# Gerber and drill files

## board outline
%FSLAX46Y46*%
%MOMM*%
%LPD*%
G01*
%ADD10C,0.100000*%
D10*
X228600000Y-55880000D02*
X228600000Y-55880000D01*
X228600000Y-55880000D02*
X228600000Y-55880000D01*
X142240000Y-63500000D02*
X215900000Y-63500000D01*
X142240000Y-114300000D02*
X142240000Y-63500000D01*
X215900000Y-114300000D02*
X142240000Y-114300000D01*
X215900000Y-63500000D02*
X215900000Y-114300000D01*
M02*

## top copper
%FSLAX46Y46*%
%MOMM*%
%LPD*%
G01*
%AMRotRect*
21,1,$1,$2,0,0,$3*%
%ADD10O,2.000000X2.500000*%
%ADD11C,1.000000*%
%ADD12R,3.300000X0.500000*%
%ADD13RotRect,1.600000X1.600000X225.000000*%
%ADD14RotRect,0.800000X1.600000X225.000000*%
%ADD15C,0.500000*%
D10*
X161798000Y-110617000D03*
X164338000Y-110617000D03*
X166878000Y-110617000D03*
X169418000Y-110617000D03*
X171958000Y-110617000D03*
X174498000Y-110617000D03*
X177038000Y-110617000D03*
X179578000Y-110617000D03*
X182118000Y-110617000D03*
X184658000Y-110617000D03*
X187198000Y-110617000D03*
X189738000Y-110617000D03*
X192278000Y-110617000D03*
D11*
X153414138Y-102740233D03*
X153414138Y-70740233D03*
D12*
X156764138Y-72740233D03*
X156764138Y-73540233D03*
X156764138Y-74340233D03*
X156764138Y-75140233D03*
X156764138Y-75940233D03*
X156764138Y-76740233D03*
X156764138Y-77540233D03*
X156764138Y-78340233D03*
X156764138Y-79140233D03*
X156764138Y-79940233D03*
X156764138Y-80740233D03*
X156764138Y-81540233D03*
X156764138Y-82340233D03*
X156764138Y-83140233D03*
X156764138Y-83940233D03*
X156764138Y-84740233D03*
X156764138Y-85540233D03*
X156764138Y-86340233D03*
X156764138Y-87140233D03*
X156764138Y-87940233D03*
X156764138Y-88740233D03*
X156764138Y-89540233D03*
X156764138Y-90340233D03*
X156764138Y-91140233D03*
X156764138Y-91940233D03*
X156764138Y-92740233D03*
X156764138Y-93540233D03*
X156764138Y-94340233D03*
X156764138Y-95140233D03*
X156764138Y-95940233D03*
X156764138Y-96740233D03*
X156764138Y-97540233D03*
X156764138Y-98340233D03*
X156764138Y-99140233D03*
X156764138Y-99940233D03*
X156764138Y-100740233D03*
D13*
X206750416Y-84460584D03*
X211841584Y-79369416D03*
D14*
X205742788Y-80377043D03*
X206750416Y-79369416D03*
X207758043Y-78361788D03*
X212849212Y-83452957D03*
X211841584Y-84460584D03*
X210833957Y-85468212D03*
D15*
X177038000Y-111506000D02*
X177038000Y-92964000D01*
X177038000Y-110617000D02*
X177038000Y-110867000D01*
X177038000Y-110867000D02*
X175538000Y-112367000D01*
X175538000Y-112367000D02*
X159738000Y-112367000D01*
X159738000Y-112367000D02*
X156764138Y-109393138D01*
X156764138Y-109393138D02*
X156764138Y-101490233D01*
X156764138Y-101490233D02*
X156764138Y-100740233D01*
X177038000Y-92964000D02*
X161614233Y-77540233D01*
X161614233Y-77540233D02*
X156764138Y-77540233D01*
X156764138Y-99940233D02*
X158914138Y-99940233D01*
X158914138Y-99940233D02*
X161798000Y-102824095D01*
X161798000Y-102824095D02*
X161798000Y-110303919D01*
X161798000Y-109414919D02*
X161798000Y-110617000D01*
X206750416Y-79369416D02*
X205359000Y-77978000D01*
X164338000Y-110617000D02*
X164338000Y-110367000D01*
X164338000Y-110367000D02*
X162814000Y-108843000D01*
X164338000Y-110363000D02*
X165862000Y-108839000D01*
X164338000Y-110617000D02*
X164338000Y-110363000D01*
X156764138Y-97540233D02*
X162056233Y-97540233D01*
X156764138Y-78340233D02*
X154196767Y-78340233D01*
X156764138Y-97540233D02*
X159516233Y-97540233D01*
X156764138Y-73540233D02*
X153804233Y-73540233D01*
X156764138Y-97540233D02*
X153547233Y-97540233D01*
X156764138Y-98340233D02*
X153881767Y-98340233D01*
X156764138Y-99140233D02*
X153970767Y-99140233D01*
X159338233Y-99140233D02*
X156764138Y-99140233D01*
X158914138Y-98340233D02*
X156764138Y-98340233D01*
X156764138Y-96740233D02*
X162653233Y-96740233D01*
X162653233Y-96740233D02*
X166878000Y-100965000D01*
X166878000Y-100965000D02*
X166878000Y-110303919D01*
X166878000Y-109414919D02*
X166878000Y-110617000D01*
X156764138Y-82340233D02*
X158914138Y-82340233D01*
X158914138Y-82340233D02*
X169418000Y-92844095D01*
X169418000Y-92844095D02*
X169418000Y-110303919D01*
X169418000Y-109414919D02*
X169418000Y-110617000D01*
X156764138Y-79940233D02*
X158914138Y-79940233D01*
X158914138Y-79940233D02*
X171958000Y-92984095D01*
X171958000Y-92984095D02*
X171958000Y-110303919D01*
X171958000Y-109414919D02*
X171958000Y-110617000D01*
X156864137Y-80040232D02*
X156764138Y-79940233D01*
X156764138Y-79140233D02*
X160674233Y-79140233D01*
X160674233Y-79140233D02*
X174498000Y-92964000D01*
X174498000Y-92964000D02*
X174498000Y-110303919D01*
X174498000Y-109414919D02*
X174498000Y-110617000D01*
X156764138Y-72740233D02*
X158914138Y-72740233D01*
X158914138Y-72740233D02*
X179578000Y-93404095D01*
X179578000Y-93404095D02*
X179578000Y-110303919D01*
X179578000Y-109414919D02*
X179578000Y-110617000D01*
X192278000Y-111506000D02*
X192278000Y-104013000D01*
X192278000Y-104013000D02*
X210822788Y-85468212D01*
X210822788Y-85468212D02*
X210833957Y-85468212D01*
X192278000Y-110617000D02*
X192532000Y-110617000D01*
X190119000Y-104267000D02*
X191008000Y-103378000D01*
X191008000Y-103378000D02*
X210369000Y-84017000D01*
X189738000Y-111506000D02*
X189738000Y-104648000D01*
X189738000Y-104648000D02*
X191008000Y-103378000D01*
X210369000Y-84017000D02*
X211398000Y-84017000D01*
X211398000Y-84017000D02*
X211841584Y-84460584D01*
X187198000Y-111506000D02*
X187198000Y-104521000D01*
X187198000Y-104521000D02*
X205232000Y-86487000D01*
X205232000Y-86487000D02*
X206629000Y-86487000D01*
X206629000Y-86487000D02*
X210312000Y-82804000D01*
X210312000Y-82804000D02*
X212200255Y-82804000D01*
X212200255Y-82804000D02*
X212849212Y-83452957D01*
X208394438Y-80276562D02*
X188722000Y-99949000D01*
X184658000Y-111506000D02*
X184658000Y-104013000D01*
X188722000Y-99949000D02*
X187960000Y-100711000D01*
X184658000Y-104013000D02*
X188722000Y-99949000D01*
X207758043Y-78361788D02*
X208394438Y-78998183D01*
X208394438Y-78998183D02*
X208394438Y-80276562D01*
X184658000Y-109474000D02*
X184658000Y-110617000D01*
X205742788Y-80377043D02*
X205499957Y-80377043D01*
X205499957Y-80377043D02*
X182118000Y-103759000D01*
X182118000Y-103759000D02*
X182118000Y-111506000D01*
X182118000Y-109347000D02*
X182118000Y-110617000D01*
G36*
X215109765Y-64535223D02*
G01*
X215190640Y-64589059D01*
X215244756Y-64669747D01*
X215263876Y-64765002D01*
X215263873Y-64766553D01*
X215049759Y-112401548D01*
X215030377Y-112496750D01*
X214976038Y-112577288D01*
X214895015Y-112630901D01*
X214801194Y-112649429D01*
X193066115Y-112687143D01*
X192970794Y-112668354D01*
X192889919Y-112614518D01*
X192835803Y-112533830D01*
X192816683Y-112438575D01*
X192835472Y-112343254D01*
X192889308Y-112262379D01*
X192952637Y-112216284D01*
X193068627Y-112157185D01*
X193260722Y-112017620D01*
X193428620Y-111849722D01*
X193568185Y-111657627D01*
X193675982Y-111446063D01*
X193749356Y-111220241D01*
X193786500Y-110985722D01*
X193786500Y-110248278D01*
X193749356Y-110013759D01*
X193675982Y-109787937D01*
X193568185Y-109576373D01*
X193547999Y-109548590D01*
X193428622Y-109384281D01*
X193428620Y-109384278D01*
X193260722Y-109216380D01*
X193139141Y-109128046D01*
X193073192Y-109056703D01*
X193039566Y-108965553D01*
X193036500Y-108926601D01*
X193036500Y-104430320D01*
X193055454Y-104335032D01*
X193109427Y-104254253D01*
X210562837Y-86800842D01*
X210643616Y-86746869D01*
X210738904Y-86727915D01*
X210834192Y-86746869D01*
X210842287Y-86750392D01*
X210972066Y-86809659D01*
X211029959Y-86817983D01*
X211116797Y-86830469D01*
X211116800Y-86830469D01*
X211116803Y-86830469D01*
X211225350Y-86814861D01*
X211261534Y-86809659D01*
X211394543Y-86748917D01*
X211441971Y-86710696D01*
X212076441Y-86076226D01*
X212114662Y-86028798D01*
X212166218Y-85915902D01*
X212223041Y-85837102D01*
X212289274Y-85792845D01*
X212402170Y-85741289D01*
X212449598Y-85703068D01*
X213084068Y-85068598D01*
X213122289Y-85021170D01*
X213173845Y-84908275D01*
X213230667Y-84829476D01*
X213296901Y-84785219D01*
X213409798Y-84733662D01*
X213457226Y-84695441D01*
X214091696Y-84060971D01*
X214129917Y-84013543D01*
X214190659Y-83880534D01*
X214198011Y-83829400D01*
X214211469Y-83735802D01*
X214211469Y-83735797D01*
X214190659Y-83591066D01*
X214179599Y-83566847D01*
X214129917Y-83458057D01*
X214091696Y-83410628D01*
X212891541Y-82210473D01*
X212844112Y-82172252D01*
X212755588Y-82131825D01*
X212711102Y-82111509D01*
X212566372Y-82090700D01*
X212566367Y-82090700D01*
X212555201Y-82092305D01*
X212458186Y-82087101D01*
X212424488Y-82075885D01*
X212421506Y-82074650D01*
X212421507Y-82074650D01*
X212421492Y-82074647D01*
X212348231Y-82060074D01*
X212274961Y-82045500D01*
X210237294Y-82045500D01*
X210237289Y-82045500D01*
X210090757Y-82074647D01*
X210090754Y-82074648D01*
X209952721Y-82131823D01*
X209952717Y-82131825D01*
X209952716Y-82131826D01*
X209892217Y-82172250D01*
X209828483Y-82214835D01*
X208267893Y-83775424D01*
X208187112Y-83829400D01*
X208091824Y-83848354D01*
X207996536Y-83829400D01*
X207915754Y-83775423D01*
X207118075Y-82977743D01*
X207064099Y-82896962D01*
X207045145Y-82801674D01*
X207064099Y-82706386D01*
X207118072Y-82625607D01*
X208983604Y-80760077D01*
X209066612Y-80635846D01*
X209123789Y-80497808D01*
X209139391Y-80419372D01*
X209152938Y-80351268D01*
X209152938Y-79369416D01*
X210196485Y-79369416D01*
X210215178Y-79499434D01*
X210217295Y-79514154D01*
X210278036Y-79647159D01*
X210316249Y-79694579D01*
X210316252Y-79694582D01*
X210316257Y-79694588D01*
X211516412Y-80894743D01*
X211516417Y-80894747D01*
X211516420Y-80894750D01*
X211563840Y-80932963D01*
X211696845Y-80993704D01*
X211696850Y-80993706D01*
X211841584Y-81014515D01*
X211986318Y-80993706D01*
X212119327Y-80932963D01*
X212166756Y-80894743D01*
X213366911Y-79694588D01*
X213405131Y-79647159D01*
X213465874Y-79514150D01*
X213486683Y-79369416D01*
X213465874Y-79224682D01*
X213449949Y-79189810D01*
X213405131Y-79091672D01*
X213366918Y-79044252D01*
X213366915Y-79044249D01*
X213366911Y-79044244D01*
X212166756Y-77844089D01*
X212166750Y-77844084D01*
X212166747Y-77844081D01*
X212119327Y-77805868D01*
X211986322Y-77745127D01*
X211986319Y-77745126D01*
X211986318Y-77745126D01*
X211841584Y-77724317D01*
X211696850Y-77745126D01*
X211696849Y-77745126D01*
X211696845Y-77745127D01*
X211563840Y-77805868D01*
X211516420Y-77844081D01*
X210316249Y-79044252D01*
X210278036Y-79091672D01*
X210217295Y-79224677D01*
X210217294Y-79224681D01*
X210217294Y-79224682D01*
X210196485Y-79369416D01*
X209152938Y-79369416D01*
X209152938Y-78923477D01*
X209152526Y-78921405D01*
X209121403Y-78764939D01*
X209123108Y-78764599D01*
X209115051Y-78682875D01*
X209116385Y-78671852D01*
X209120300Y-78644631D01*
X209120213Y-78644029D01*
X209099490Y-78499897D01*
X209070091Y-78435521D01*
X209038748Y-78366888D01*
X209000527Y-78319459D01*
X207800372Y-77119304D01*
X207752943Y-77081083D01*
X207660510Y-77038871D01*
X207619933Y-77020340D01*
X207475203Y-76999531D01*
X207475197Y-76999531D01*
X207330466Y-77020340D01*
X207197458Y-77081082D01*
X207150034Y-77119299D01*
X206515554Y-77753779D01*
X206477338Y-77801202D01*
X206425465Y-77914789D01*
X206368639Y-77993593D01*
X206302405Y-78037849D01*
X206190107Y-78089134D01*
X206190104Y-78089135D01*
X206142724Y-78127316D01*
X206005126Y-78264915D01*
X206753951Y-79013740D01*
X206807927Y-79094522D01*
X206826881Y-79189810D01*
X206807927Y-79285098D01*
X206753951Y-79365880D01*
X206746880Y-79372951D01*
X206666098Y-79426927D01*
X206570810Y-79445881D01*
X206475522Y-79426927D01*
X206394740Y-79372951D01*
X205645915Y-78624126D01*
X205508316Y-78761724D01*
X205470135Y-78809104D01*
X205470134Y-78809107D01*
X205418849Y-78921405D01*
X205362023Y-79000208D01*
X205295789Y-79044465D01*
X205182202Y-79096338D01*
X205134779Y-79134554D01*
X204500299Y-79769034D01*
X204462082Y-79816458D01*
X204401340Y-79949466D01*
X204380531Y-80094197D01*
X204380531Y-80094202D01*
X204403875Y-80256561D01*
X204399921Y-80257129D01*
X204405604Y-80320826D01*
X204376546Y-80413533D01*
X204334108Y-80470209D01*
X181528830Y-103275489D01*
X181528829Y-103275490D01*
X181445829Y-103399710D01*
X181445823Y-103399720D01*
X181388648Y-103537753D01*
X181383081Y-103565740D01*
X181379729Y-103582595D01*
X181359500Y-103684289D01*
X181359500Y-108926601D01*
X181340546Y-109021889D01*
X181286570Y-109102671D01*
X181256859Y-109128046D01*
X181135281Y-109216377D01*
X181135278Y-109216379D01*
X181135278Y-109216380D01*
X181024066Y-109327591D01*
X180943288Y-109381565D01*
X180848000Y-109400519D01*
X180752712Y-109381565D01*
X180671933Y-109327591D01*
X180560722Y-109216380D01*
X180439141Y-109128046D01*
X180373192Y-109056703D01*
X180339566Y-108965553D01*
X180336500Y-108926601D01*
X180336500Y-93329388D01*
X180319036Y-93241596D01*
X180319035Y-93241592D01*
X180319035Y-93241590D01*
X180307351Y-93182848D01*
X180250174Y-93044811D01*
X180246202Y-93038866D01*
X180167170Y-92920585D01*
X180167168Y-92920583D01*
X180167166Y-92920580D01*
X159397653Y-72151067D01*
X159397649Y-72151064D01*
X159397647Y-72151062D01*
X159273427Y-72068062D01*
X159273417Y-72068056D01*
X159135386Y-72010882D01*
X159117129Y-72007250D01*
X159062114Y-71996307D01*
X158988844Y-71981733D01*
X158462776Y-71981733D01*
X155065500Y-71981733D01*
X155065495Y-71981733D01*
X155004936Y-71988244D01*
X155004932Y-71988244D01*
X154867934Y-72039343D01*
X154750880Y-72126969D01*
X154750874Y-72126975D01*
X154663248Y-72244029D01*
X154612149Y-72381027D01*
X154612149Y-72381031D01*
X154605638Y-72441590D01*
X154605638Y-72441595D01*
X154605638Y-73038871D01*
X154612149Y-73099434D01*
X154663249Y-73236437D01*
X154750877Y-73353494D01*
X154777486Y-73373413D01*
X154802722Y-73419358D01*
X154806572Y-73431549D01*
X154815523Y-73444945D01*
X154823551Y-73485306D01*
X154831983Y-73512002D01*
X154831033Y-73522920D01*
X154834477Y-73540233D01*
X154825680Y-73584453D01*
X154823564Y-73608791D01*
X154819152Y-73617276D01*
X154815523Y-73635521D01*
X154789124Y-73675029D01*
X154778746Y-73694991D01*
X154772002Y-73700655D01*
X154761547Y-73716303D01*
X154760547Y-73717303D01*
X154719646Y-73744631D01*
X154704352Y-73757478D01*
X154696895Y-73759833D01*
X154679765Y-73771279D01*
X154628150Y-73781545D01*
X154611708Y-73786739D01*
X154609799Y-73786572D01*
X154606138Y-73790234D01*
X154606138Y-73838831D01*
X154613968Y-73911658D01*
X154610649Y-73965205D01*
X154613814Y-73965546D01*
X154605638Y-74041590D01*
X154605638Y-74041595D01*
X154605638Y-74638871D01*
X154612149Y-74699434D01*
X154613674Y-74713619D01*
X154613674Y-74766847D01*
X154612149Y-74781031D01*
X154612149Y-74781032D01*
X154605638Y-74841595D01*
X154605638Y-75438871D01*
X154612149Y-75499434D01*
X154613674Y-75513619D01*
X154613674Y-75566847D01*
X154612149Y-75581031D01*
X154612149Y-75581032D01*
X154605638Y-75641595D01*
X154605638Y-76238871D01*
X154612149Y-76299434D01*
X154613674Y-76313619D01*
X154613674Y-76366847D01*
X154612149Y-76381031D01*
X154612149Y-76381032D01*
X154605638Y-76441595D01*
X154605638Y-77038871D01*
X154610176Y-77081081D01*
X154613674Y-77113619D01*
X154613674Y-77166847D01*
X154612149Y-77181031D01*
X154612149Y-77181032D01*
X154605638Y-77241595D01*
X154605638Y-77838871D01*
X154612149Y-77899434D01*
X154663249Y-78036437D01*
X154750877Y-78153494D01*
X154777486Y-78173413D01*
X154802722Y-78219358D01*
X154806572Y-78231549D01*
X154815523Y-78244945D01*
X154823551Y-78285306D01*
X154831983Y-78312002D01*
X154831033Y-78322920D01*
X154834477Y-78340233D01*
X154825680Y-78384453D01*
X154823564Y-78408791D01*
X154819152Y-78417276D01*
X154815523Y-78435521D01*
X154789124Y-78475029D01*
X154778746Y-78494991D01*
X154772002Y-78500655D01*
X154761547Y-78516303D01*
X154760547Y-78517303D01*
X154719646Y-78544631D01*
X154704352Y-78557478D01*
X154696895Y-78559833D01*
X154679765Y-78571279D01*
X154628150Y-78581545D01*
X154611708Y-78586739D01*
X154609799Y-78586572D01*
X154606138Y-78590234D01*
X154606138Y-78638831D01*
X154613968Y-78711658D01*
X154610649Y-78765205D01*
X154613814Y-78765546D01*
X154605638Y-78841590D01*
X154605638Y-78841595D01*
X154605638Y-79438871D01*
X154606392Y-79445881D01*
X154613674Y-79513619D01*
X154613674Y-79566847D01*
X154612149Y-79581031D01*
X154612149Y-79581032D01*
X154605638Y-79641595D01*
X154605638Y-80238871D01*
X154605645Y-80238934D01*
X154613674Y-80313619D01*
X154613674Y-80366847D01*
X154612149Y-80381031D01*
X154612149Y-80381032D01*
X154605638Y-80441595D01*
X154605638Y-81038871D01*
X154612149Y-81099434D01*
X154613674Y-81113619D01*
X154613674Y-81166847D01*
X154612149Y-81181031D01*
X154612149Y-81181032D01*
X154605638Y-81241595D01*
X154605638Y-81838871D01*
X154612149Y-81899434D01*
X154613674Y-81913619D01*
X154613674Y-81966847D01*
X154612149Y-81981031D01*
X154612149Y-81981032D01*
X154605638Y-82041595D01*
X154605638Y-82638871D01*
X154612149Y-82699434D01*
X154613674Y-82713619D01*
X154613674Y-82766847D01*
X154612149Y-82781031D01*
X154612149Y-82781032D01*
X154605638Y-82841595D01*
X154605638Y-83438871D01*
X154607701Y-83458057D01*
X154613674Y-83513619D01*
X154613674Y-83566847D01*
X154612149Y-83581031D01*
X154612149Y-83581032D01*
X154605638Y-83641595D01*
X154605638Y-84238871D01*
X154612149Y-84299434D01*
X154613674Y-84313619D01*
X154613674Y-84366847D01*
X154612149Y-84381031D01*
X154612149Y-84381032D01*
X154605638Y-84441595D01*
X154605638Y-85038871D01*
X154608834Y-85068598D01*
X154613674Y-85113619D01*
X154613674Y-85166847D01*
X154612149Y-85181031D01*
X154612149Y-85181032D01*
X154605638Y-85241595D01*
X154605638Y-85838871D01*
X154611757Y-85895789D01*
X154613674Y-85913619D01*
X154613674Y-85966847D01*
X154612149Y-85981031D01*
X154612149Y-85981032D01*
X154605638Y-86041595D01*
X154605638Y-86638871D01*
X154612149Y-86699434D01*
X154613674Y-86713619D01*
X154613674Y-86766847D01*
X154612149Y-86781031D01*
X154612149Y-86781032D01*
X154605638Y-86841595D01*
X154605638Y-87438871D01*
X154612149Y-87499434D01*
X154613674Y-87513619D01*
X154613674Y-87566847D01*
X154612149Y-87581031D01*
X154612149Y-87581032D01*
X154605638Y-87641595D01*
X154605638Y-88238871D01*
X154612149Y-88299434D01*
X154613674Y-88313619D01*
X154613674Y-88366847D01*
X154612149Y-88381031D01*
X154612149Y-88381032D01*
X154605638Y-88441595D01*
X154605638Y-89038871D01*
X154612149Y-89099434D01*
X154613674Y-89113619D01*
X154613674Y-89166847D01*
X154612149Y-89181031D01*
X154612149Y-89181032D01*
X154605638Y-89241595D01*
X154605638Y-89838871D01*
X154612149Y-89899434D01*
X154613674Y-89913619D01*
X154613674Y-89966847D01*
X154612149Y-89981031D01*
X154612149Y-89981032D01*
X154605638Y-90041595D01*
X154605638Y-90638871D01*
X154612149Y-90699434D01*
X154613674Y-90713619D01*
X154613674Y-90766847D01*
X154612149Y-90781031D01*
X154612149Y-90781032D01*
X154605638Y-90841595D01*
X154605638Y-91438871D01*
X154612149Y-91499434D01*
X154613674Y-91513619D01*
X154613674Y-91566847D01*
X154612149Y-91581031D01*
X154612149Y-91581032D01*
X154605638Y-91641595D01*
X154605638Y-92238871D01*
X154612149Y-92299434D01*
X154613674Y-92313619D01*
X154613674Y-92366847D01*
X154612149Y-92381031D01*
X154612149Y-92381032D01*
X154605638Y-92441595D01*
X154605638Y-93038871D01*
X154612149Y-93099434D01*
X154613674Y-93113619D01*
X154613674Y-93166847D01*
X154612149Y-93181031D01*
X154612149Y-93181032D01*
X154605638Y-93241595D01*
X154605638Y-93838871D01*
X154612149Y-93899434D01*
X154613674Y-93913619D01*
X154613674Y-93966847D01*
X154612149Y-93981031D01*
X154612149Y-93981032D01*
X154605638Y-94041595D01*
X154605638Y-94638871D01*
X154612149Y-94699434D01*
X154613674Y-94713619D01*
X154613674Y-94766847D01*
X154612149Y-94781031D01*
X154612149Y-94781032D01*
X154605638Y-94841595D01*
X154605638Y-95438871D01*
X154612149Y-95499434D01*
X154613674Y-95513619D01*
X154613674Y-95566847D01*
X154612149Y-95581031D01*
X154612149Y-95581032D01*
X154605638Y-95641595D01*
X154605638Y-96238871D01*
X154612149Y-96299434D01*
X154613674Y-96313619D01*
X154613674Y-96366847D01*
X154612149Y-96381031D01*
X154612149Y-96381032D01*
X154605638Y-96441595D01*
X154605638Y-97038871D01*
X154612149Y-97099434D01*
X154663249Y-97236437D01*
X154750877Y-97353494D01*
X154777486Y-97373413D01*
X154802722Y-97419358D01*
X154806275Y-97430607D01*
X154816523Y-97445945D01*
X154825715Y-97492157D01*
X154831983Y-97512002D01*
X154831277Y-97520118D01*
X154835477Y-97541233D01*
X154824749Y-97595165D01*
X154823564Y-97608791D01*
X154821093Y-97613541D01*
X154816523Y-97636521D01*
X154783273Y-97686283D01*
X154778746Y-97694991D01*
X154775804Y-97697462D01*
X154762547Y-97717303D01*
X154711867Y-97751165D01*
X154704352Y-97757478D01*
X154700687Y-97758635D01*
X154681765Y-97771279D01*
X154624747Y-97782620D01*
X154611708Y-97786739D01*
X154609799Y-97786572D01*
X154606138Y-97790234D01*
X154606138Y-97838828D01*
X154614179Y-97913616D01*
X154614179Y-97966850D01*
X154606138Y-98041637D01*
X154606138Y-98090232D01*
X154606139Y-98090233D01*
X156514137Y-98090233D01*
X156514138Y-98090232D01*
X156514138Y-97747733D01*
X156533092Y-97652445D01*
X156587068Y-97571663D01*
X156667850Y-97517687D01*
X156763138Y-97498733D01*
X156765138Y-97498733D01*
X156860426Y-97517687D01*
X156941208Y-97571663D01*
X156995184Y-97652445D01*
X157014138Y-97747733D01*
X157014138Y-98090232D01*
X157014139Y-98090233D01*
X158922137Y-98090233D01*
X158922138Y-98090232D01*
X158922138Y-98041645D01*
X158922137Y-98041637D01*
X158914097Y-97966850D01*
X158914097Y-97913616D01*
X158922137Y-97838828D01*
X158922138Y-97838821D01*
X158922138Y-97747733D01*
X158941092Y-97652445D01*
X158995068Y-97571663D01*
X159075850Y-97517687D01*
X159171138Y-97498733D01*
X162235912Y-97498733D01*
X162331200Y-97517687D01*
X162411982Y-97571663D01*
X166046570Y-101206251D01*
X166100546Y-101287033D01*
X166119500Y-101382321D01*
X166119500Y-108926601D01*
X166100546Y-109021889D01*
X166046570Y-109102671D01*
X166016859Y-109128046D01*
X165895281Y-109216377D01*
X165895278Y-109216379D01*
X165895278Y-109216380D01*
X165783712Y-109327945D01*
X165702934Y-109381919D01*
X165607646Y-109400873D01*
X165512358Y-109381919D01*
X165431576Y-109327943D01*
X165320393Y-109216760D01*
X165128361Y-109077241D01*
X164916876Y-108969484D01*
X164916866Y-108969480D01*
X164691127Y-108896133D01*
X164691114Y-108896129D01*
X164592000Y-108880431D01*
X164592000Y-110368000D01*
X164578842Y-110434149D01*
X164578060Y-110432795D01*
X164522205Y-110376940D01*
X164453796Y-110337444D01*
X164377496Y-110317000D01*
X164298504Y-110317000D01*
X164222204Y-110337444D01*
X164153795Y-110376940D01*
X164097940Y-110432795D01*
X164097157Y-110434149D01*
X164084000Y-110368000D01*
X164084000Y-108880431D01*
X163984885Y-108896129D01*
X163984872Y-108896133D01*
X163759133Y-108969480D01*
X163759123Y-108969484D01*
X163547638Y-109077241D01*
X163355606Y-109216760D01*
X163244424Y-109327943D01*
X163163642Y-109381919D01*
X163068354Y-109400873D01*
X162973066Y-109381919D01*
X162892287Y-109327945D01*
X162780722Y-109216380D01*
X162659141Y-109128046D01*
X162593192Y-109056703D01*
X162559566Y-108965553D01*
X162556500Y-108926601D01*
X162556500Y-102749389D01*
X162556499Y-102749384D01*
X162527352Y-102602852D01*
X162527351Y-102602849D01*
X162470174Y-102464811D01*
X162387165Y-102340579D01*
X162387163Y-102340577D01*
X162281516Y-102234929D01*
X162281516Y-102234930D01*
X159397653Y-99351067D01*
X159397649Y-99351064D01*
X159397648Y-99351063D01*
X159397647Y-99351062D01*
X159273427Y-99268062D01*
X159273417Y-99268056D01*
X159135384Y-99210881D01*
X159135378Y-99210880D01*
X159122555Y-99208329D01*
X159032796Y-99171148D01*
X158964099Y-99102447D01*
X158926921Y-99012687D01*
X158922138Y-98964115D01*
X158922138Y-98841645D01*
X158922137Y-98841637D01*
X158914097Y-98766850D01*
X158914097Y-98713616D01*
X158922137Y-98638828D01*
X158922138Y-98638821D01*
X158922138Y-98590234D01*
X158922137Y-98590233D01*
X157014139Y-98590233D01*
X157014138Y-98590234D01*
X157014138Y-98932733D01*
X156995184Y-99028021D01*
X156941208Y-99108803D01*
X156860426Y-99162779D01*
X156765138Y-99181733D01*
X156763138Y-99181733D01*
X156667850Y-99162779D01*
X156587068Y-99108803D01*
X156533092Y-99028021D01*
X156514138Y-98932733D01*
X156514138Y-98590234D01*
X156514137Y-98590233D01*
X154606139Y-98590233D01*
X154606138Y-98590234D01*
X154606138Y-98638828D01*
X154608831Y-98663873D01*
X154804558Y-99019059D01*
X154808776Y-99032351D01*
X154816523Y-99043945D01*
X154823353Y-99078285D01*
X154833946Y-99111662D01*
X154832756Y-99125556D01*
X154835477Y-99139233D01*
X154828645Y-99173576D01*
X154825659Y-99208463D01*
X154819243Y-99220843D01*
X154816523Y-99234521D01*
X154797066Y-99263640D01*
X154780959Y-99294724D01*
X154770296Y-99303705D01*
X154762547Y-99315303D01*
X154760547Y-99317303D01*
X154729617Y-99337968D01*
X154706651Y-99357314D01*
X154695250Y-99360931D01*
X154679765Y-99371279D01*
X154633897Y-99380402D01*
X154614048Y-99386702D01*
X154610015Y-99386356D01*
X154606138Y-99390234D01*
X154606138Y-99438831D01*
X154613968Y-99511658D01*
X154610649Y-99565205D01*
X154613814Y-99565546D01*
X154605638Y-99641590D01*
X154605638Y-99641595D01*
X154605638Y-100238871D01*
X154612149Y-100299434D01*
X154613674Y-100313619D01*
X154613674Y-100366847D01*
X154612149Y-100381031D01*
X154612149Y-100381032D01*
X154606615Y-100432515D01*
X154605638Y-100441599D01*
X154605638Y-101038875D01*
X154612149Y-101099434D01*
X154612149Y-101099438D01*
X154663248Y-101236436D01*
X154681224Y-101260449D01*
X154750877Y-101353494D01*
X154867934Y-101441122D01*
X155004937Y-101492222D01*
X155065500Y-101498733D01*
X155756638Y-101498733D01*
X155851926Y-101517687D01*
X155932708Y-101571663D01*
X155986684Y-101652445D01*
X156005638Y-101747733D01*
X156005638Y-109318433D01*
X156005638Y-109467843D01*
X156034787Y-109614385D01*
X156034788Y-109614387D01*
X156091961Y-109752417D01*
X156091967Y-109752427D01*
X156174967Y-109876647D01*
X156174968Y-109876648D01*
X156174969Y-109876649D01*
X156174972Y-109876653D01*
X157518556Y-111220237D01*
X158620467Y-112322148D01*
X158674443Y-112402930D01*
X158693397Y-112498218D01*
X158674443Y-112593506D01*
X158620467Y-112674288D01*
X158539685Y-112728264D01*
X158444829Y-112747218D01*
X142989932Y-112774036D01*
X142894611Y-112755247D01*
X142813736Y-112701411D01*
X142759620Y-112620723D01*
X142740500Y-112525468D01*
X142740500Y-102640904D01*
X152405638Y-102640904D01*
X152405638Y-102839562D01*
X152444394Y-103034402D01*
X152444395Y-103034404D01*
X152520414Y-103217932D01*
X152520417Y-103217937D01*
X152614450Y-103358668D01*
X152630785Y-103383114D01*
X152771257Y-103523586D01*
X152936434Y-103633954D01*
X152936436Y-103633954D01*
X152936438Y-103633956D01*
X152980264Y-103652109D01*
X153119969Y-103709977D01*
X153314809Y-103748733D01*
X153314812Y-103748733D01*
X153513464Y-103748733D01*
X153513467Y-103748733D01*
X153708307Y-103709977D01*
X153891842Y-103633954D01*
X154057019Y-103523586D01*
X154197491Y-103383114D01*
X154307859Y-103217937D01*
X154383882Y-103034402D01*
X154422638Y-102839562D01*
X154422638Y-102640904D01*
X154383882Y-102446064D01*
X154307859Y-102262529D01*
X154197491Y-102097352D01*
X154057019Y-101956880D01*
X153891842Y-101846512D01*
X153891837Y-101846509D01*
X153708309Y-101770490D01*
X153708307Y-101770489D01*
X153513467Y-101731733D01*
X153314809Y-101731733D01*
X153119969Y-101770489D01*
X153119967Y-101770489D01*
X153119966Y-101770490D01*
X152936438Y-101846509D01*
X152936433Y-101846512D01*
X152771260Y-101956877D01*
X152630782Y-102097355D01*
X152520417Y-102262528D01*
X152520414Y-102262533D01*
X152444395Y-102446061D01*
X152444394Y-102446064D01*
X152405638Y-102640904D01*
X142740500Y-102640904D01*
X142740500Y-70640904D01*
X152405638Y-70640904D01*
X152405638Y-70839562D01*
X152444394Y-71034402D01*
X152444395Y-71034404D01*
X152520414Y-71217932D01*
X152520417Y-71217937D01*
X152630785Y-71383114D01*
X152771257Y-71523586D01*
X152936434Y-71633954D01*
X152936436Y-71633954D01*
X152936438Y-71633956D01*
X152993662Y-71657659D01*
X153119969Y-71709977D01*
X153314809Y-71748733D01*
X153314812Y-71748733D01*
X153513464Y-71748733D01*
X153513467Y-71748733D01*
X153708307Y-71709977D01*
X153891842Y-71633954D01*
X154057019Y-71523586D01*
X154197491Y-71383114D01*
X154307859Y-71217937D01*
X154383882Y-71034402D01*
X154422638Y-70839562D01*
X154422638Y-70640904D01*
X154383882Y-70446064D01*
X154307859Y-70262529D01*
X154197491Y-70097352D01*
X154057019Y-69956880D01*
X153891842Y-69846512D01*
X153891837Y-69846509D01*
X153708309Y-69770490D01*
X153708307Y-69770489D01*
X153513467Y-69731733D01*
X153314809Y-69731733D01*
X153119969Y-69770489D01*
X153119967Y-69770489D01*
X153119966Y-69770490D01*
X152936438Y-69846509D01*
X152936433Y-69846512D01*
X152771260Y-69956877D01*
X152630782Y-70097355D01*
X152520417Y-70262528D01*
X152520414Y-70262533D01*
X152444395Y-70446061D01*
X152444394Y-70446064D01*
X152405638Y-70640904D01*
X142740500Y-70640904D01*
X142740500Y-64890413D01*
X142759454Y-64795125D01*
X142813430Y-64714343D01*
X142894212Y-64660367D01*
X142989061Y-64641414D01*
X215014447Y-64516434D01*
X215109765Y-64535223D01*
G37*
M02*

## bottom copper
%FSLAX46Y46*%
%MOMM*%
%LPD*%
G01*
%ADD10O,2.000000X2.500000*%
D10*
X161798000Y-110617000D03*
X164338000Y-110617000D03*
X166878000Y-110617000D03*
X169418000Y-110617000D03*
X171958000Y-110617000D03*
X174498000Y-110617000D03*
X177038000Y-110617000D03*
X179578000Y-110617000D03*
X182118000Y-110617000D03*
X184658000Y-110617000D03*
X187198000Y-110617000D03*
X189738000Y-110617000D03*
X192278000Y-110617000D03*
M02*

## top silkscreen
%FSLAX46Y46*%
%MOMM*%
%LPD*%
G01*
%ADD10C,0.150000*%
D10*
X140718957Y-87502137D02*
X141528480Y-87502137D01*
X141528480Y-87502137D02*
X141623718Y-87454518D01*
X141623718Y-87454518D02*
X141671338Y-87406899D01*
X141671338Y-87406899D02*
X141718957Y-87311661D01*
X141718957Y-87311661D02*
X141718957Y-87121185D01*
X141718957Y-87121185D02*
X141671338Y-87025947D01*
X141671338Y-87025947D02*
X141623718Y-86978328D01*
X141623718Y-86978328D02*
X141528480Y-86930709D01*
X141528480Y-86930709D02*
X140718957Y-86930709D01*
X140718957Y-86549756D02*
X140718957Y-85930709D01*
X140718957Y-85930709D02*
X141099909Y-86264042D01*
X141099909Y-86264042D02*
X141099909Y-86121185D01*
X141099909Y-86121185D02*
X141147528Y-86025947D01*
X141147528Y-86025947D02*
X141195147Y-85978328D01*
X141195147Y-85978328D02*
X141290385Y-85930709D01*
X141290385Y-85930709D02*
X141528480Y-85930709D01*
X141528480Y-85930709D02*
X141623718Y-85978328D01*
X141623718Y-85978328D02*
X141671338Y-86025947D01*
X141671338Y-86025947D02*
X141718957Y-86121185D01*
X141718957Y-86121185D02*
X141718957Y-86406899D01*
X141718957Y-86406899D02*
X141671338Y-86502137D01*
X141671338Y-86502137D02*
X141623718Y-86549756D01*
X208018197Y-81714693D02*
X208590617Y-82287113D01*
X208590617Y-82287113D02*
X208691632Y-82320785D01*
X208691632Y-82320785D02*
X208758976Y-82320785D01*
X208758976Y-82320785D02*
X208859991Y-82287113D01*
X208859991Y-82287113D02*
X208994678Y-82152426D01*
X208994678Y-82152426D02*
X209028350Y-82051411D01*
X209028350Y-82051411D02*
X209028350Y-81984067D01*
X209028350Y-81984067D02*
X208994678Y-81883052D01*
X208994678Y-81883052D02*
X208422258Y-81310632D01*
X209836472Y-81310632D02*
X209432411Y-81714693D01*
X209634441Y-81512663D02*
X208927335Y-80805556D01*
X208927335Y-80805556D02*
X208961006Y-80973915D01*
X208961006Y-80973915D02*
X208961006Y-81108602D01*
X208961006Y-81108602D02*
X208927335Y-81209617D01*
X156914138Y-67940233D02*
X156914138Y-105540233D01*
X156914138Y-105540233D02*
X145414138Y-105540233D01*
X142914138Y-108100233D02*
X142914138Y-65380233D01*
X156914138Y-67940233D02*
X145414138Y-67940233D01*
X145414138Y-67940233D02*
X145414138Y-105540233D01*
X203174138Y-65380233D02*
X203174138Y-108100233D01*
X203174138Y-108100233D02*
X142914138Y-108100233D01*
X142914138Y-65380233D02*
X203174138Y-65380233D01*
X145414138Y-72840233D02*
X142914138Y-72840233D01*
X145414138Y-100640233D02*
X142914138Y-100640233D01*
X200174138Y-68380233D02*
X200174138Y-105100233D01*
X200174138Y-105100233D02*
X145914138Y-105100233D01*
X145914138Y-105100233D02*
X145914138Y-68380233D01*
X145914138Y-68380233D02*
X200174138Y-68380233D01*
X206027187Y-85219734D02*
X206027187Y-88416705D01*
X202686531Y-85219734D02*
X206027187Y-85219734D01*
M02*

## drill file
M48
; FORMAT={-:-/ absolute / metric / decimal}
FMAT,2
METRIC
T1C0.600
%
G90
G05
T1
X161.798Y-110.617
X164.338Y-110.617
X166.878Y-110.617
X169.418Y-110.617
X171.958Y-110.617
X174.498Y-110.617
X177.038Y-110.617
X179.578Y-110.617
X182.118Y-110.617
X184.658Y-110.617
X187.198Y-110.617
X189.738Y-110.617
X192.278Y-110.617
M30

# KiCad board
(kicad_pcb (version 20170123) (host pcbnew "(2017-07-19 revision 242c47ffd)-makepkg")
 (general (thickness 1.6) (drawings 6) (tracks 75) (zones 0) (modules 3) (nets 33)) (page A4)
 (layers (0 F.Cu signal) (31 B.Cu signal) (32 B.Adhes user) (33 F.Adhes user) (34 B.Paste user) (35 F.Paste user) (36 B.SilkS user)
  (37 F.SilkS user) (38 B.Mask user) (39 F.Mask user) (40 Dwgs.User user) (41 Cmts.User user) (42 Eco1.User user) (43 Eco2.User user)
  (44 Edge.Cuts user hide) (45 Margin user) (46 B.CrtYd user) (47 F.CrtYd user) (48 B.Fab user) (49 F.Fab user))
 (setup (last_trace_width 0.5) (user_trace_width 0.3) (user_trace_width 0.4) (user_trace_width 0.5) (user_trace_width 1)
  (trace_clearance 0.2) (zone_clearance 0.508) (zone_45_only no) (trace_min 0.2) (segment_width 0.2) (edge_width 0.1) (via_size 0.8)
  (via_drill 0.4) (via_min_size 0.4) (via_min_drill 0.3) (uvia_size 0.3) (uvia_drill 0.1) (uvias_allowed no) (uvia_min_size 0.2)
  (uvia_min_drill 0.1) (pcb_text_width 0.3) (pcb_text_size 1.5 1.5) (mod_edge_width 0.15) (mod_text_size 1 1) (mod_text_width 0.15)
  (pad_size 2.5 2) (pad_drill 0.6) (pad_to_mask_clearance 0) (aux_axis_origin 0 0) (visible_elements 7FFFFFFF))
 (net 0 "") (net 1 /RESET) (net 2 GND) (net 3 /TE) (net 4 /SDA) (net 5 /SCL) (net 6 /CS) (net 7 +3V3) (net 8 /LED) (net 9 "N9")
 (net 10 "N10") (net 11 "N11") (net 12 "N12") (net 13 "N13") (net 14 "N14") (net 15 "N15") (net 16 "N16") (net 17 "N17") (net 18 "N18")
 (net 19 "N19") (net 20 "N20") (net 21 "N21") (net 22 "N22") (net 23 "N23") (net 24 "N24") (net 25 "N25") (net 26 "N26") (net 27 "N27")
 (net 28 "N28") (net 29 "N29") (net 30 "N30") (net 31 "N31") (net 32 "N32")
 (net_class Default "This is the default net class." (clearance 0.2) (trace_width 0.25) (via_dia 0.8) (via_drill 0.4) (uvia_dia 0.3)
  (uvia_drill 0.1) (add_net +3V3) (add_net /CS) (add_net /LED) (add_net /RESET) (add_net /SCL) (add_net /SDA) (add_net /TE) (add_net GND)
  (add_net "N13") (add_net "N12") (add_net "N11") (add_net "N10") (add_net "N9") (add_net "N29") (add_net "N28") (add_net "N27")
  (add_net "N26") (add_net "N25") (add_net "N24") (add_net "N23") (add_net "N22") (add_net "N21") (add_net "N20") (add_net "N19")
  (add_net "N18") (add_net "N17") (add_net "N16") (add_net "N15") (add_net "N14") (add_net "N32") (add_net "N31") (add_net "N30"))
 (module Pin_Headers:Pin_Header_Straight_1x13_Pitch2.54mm (layer B.Cu) (at 192.278 110.617 90)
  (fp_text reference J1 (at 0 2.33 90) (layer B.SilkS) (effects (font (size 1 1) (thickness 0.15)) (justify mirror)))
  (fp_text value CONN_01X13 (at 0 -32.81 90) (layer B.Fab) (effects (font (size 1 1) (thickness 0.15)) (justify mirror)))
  (pad 13 thru_hole oval (at 0 -30.48 90) (size 2.5 2) (drill 0.6) (layers *.Cu *.Mask) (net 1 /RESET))
  (pad 12 thru_hole oval (at 0 -27.94 90) (size 2.5 2) (drill 0.6) (layers *.Cu *.Mask) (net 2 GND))
  (pad 11 thru_hole oval (at 0 -25.4 90) (size 2.5 2) (drill 0.6) (layers *.Cu *.Mask) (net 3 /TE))
  (pad 10 thru_hole oval (at 0 -22.86 90) (size 2.5 2) (drill 0.6) (layers *.Cu *.Mask) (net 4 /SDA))
  (pad 9 thru_hole oval (at 0 -20.32 90) (size 2.5 2) (drill 0.6) (layers *.Cu *.Mask) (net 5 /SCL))
  (pad 8 thru_hole oval (at 0 -17.78 90) (size 2.5 2) (drill 0.6) (layers *.Cu *.Mask) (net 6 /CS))
  (pad 7 thru_hole oval (at 0 -15.24 90) (size 2.5 2) (drill 0.6) (layers *.Cu *.Mask) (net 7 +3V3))
  (pad 6 thru_hole oval (at 0 -12.7 90) (size 2.5 2) (drill 0.6) (layers *.Cu *.Mask) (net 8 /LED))
  (pad 5 thru_hole oval (at 0 -10.16 90) (size 2.5 2) (drill 0.6) (layers *.Cu *.Mask) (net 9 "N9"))
  (pad 4 thru_hole oval (at 0 -7.62 90) (size 2.5 2) (drill 0.6) (layers *.Cu *.Mask) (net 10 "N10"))
  (pad 3 thru_hole oval (at 0 -5.08 90) (size 2.5 2) (drill 0.6) (layers *.Cu *.Mask) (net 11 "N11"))
  (pad 2 thru_hole oval (at 0 -2.54 90) (size 2.5 2) (drill 0.6) (layers *.Cu *.Mask) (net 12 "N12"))
  (pad 1 thru_hole oval (at 0 0 90) (size 2.5 2) (drill 0.6) (layers *.Cu *.Mask) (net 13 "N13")))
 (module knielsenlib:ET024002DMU (layer F.Cu) (at 156.764138 86.740233 270)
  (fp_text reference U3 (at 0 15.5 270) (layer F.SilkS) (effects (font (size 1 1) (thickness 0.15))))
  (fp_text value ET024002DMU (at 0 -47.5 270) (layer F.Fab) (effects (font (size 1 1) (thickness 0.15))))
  (fp_line (start -18.8 -0.15) (end 18.8 -0.15) (layer F.SilkS) (width 0.15))
  (fp_line (start 18.8 -0.15) (end 18.8 11.35) (layer F.SilkS) (width 0.15))
  (fp_line (start 21.36 13.85) (end -21.36 13.85) (layer F.SilkS) (width 0.15))
  (fp_line (start -18.8 -0.15) (end -18.8 11.35) (layer F.SilkS) (width 0.15))
  (fp_line (start -18.8 11.35) (end 18.8 11.35) (layer F.SilkS) (width 0.15))
  (fp_line (start -21.36 -46.41) (end 21.36 -46.41) (layer F.SilkS) (width 0.15))
  (fp_line (start 21.36 -46.41) (end 21.36 13.85) (layer F.SilkS) (width 0.15))
  (fp_line (start -21.36 13.85) (end -21.36 -46.41) (layer F.SilkS) (width 0.15))
  (fp_line (start -13.9 11.35) (end -13.9 13.85) (layer F.SilkS) (width 0.15))
  (fp_line (start 13.9 11.35) (end 13.9 13.85) (layer F.SilkS) (width 0.15))
  (fp_line (start -18.36 -43.41) (end 18.36 -43.41) (layer F.SilkS) (width 0.15))
  (fp_line (start 18.36 -43.41) (end 18.36 10.85) (layer F.SilkS) (width 0.15))
  (fp_line (start 18.36 10.85) (end -18.36 10.85) (layer F.SilkS) (width 0.15))
  (fp_line (start -18.36 10.85) (end -18.36 -43.41) (layer F.SilkS) (width 0.15))
  (pad "" smd circle (at 16 3.35 270) (size 1 1) (layers F.Cu F.Paste F.Mask))
  (pad "" smd circle (at -16 3.35 270) (size 1 1) (layers F.Cu F.Paste F.Mask))
  (pad 36 smd rect (at -14 0 90) (size 0.5 3.3) (layers F.Cu F.Paste F.Mask) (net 8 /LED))
  (pad 35 smd rect (at -13.2 0 90) (size 0.5 3.3) (layers F.Cu F.Paste F.Mask) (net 2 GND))
  (pad 34 smd rect (at -12.4 0 90) (size 0.5 3.3) (layers F.Cu F.Paste F.Mask))
  (pad 33 smd rect (at -11.6 0 90) (size 0.5 3.3) (layers F.Cu F.Paste F.Mask))
  (pad 32 smd rect (at -10.8 0 90) (size 0.5 3.3) (layers F.Cu F.Paste F.Mask))
  (pad 31 smd rect (at -10 0 90) (size 0.5 3.3) (layers F.Cu F.Paste F.Mask))
  (pad 30 smd rect (at -9.2 0 90) (size 0.5 3.3) (layers F.Cu F.Paste F.Mask) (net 7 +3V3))
  (pad 29 smd rect (at -8.4 0 90) (size 0.5 3.3) (layers F.Cu F.Paste F.Mask) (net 2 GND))
  (pad 28 smd rect (at -7.6 0 90) (size 0.5 3.3) (layers F.Cu F.Paste F.Mask) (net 6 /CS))
  (pad 27 smd rect (at -6.8 0 90) (size 0.5 3.3) (layers F.Cu F.Paste F.Mask) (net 5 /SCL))
  (pad 26 smd rect (at -6 0 90) (size 0.5 3.3) (layers F.Cu F.Paste F.Mask) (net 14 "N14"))
  (pad 25 smd rect (at -5.2 0 90) (size 0.5 3.3) (layers F.Cu F.Paste F.Mask) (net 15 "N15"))
  (pad 24 smd rect (at -4.4 0 90) (size 0.5 3.3) (layers F.Cu F.Paste F.Mask) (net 4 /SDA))
  (pad 23 smd rect (at -3.6 0 90) (size 0.5 3.3) (layers F.Cu F.Paste F.Mask) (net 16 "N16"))
  (pad 22 smd rect (at -2.8 0 90) (size 0.5 3.3) (layers F.Cu F.Paste F.Mask) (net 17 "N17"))
  (pad 21 smd rect (at -2 0 90) (size 0.5 3.3) (layers F.Cu F.Paste F.Mask) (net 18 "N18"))
  (pad 20 smd rect (at -1.2 0 90) (size 0.5 3.3) (layers F.Cu F.Paste F.Mask) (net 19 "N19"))
  (pad 19 smd rect (at -0.4 0 90) (size 0.5 3.3) (layers F.Cu F.Paste F.Mask) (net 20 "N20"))
  (pad 18 smd rect (at 0.4 0 90) (size 0.5 3.3) (layers F.Cu F.Paste F.Mask) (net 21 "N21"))
  (pad 17 smd rect (at 1.2 0 90) (size 0.5 3.3) (layers F.Cu F.Paste F.Mask) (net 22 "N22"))
  (pad 16 smd rect (at 2 0 90) (size 0.5 3.3) (layers F.Cu F.Paste F.Mask) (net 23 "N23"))
  (pad 15 smd rect (at 2.8 0 90) (size 0.5 3.3) (layers F.Cu F.Paste F.Mask) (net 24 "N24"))
  (pad 14 smd rect (at 3.6 0 90) (size 0.5 3.3) (layers F.Cu F.Paste F.Mask) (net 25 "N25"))
  (pad 13 smd rect (at 4.4 0 90) (size 0.5 3.3) (layers F.Cu F.Paste F.Mask) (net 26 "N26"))
  (pad 12 smd rect (at 5.2 0 90) (size 0.5 3.3) (layers F.Cu F.Paste F.Mask) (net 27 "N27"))
  (pad 11 smd rect (at 6 0 90) (size 0.5 3.3) (layers F.Cu F.Paste F.Mask) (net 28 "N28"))
  (pad 10 smd rect (at 6.8 0 90) (size 0.5 3.3) (layers F.Cu F.Paste F.Mask) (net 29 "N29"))
  (pad 9 smd rect (at 7.6 0 90) (size 0.5 3.3) (layers F.Cu F.Paste F.Mask) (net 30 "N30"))
  (pad 8 smd rect (at 8.4 0 90) (size 0.5 3.3) (layers F.Cu F.Paste F.Mask) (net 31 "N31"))
  (pad 7 smd rect (at 9.2 0 90) (size 0.5 3.3) (layers F.Cu F.Paste F.Mask) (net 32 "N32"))
  (pad 6 smd rect (at 10 0 90) (size 0.5 3.3) (layers F.Cu F.Paste F.Mask) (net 3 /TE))
  (pad 5 smd rect (at 10.8 0 90) (size 0.5 3.3) (layers F.Cu F.Paste F.Mask) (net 2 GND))
  (pad 4 smd rect (at 11.6 0 90) (size 0.5 3.3) (layers F.Cu F.Paste F.Mask) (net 2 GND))
  (pad 3 smd rect (at 12.4 0 90) (size 0.5 3.3) (layers F.Cu F.Paste F.Mask) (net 2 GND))
  (pad 2 smd rect (at 13.2 0 90) (size 0.5 3.3) (layers F.Cu F.Paste F.Mask) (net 1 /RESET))
  (pad 1 smd rect (at 14 0 90) (size 0.5 3.3) (layers F.Cu F.Paste F.Mask) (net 7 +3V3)))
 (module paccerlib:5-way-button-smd (layer F.Cu) (at 209.296 81.915 225)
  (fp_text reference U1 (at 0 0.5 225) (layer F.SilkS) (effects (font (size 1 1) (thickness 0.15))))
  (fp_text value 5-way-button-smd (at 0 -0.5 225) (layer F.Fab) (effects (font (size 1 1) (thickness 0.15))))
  (fp_line (start 4.6482 -0.0254) (end 6.9088 -2.286) (layer F.SilkS) (width 0.15))
  (fp_line (start 7.0104 2.336801) (end 4.6482 -0.0254) (layer F.SilkS) (width 0.15))
  (pad 7 smd rect (at 3.599999 0 225) (size 1.6 1.6) (layers F.Cu F.Paste F.Mask))
  (pad 7 smd rect (at -3.599999 0 225) (size 1.6 1.6) (layers F.Cu F.Paste F.Mask))
  (pad 6 smd rect (at 1.425 3.6 225) (size 0.8 1.6) (layers F.Cu F.Paste F.Mask) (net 9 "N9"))
  (pad 5 smd rect (at 0 3.599999 225) (size 0.8 1.6) (layers F.Cu F.Paste F.Mask) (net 2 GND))
  (pad 4 smd rect (at -1.425 3.6 225) (size 0.8 1.6) (layers F.Cu F.Paste F.Mask) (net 10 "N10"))
  (pad 3 smd rect (at -1.425 -3.6 225) (size 0.8 1.6) (layers F.Cu F.Paste F.Mask) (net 11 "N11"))
  (pad 2 smd rect (at 0 -3.599999 225) (size 0.8 1.6) (layers F.Cu F.Paste F.Mask) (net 12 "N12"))
  (pad 1 smd rect (at 1.425 -3.6 225) (size 0.8 1.6) (layers F.Cu F.Paste F.Mask) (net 13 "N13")))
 (gr_line (start 228.6 55.88) (end 228.6 55.88) (layer Edge.Cuts) (width 0.1))
 (gr_line (start 228.6 55.88) (end 228.6 55.88) (layer Edge.Cuts) (width 0.1))
 (gr_line (start 142.24 63.5) (end 215.9 63.5) (layer Edge.Cuts) (width 0.1))
 (gr_line (start 142.24 114.3) (end 142.24 63.5) (layer Edge.Cuts) (width 0.1))
 (gr_line (start 215.9 114.3) (end 142.24 114.3) (layer Edge.Cuts) (width 0.1))
 (gr_line (start 215.9 63.5) (end 215.9 114.3) (layer Edge.Cuts) (width 0.1))
 (segment (start 177.038 111.506) (end 177.038 92.964) (width 0.5) (layer F.Cu) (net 7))
 (segment (start 177.038 110.617) (end 177.038 110.867) (width 0.5) (layer F.Cu) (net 7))
 (segment (start 177.038 110.867) (end 175.538 112.367) (width 0.5) (layer F.Cu) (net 7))
 (segment (start 175.538 112.367) (end 159.738 112.367) (width 0.5) (layer F.Cu) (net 7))
 (segment (start 159.738 112.367) (end 156.764138 109.393138) (width 0.5) (layer F.Cu) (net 7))
 (segment (start 156.764138 109.393138) (end 156.764138 101.490233) (width 0.5) (layer F.Cu) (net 7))
 (segment (start 156.764138 101.490233) (end 156.764138 100.740233) (width 0.5) (layer F.Cu) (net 7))
 (segment (start 177.038 92.964) (end 161.614233 77.540233) (width 0.5) (layer F.Cu) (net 7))
 (segment (start 161.614233 77.540233) (end 156.764138 77.540233) (width 0.5) (layer F.Cu) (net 7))
 (segment (start 156.764138 99.940233) (end 158.914138 99.940233) (width 0.5) (layer F.Cu) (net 1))
 (segment (start 158.914138 99.940233) (end 161.798 102.824095) (width 0.5) (layer F.Cu) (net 1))
 (segment (start 161.798 102.824095) (end 161.798 110.303919) (width 0.5) (layer F.Cu) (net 1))
 (segment (start 161.798 109.414919) (end 161.798 110.617) (width 0.5) (layer F.Cu) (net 1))
 (segment (start 206.750416 79.369416) (end 205.359 77.978) (width 0.5) (layer F.Cu) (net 2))
 (segment (start 164.338 110.617) (end 164.338 110.367) (width 0.5) (layer F.Cu) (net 2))
 (segment (start 164.338 110.367) (end 162.814 108.843) (width 0.5) (layer F.Cu) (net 2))
 (segment (start 164.338 110.363) (end 165.862 108.839) (width 0.5) (layer F.Cu) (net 2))
 (segment (start 164.338 110.617) (end 164.338 110.363) (width 0.5) (layer F.Cu) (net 2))
 (segment (start 156.764138 97.540233) (end 162.056233 97.540233) (width 0.5) (layer F.Cu) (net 2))
 (segment (start 156.764138 78.340233) (end 154.196767 78.340233) (width 0.5) (layer F.Cu) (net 2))
 (segment (start 156.764138 97.540233) (end 159.516233 97.540233) (width 0.5) (layer F.Cu) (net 2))
 (segment (start 156.764138 73.540233) (end 153.804233 73.540233) (width 0.5) (layer F.Cu) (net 2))
 (segment (start 156.764138 97.540233) (end 153.547233 97.540233) (width 0.5) (layer F.Cu) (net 2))
 (segment (start 156.764138 98.340233) (end 153.881767 98.340233) (width 0.5) (layer F.Cu) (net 2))
 (segment (start 156.764138 99.140233) (end 153.970767 99.140233) (width 0.5) (layer F.Cu) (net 2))
 (segment (start 159.338233 99.140233) (end 156.764138 99.140233) (width 0.5) (layer F.Cu) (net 2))
 (segment (start 158.914138 98.340233) (end 156.764138 98.340233) (width 0.5) (layer F.Cu) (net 2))
 (segment (start 156.764138 96.740233) (end 162.653233 96.740233) (width 0.5) (layer F.Cu) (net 3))
 (segment (start 162.653233 96.740233) (end 166.878 100.965) (width 0.5) (layer F.Cu) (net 3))
 (segment (start 166.878 100.965) (end 166.878 110.303919) (width 0.5) (layer F.Cu) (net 3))
 (segment (start 166.878 109.414919) (end 166.878 110.617) (width 0.5) (layer F.Cu) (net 3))
 (segment (start 156.764138 82.340233) (end 158.914138 82.340233) (width 0.5) (layer F.Cu) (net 4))
 (segment (start 158.914138 82.340233) (end 169.418 92.844095) (width 0.5) (layer F.Cu) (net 4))
 (segment (start 169.418 92.844095) (end 169.418 110.303919) (width 0.5) (layer F.Cu) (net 4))
 (segment (start 169.418 109.414919) (end 169.418 110.617) (width 0.5) (layer F.Cu) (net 4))
 (segment (start 156.764138 79.940233) (end 158.914138 79.940233) (width 0.5) (layer F.Cu) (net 5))
 (segment (start 158.914138 79.940233) (end 171.958 92.984095) (width 0.5) (layer F.Cu) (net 5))
 (segment (start 171.958 92.984095) (end 171.958 110.303919) (width 0.5) (layer F.Cu) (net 5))
 (segment (start 171.958 109.414919) (end 171.958 110.617) (width 0.5) (layer F.Cu) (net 5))
 (segment (start 156.864137 80.040232) (end 156.764138 79.940233) (width 0.5) (layer F.Cu) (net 5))
 (segment (start 156.764138 79.140233) (end 160.674233 79.140233) (width 0.5) (layer F.Cu) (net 6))
 (segment (start 160.674233 79.140233) (end 174.498 92.964) (width 0.5) (layer F.Cu) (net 6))
 (segment (start 174.498 92.964) (end 174.498 110.303919) (width 0.5) (layer F.Cu) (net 6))
 (segment (start 174.498 109.414919) (end 174.498 110.617) (width 0.5) (layer F.Cu) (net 6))
 (segment (start 156.764138 72.740233) (end 158.914138 72.740233) (width 0.5) (layer F.Cu) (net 8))
 (segment (start 158.914138 72.740233) (end 179.578 93.404095) (width 0.5) (layer F.Cu) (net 8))
 (segment (start 179.578 93.404095) (end 179.578 110.303919) (width 0.5) (layer F.Cu) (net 8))
 (segment (start 179.578 109.414919) (end 179.578 110.617) (width 0.5) (layer F.Cu) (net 8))
 (segment (start 192.278 111.506) (end 192.278 104.013) (width 0.5) (layer F.Cu) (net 13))
 (segment (start 192.278 104.013) (end 210.822788 85.468212) (width 0.5) (layer F.Cu) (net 13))
 (segment (start 210.822788 85.468212) (end 210.833957 85.468212) (width 0.5) (layer F.Cu) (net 13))
 (segment (start 192.278 110.617) (end 192.532 110.617) (width 0.5) (layer F.Cu) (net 13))
 (segment (start 190.119 104.267) (end 191.008 103.378) (width 0.5) (layer F.Cu) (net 12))
 (segment (start 191.008 103.378) (end 210.369 84.017) (width 0.5) (layer F.Cu) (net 12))
 (segment (start 189.738 111.506) (end 189.738 104.648) (width 0.5) (layer F.Cu) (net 12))
 (segment (start 189.738 104.648) (end 191.008 103.378) (width 0.5) (layer F.Cu) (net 12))
 (segment (start 210.369 84.017) (end 211.398 84.017) (width 0.5) (layer F.Cu) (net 12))
 (segment (start 211.398 84.017) (end 211.841584 84.460584) (width 0.5) (layer F.Cu) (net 12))
 (segment (start 187.198 111.506) (end 187.198 104.521) (width 0.5) (layer F.Cu) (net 11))
 (segment (start 187.198 104.521) (end 205.232 86.487) (width 0.5) (layer F.Cu) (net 11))
 (segment (start 205.232 86.487) (end 206.629 86.487) (width 0.5) (layer F.Cu) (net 11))
 (segment (start 206.629 86.487) (end 210.312 82.804) (width 0.5) (layer F.Cu) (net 11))
 (segment (start 210.312 82.804) (end 212.200255 82.804) (width 0.5) (layer F.Cu) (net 11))
 (segment (start 212.200255 82.804) (end 212.849212 83.452957) (width 0.5) (layer F.Cu) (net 11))
 (segment (start 208.394438 80.276562) (end 188.722 99.949) (width 0.5) (layer F.Cu) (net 10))
 (segment (start 184.658 111.506) (end 184.658 104.013) (width 0.5) (layer F.Cu) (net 10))
 (segment (start 188.722 99.949) (end 187.96 100.711) (width 0.5) (layer F.Cu) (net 10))
 (segment (start 184.658 104.013) (end 188.722 99.949) (width 0.5) (layer F.Cu) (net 10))
 (segment (start 207.758043 78.361788) (end 208.394438 78.998183) (width 0.5) (layer F.Cu) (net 10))
 (segment (start 208.394438 78.998183) (end 208.394438 80.276562) (width 0.5) (layer F.Cu) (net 10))
 (segment (start 184.658 109.474) (end 184.658 110.617) (width 0.5) (layer F.Cu) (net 10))
 (segment (start 205.742788 80.377043) (end 205.499957 80.377043) (width 0.5) (layer F.Cu) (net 9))
 (segment (start 205.499957 80.377043) (end 182.118 103.759) (width 0.5) (layer F.Cu) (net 9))
 (segment (start 182.118 103.759) (end 182.118 111.506) (width 0.5) (layer F.Cu) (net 9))
 (segment (start 182.118 109.347) (end 182.118 110.617) (width 0.5) (layer F.Cu) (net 9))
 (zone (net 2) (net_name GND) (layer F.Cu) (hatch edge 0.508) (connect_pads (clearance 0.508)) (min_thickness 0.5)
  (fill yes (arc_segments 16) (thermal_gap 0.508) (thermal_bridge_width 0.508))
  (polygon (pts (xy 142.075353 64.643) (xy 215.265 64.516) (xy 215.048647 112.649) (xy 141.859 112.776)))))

